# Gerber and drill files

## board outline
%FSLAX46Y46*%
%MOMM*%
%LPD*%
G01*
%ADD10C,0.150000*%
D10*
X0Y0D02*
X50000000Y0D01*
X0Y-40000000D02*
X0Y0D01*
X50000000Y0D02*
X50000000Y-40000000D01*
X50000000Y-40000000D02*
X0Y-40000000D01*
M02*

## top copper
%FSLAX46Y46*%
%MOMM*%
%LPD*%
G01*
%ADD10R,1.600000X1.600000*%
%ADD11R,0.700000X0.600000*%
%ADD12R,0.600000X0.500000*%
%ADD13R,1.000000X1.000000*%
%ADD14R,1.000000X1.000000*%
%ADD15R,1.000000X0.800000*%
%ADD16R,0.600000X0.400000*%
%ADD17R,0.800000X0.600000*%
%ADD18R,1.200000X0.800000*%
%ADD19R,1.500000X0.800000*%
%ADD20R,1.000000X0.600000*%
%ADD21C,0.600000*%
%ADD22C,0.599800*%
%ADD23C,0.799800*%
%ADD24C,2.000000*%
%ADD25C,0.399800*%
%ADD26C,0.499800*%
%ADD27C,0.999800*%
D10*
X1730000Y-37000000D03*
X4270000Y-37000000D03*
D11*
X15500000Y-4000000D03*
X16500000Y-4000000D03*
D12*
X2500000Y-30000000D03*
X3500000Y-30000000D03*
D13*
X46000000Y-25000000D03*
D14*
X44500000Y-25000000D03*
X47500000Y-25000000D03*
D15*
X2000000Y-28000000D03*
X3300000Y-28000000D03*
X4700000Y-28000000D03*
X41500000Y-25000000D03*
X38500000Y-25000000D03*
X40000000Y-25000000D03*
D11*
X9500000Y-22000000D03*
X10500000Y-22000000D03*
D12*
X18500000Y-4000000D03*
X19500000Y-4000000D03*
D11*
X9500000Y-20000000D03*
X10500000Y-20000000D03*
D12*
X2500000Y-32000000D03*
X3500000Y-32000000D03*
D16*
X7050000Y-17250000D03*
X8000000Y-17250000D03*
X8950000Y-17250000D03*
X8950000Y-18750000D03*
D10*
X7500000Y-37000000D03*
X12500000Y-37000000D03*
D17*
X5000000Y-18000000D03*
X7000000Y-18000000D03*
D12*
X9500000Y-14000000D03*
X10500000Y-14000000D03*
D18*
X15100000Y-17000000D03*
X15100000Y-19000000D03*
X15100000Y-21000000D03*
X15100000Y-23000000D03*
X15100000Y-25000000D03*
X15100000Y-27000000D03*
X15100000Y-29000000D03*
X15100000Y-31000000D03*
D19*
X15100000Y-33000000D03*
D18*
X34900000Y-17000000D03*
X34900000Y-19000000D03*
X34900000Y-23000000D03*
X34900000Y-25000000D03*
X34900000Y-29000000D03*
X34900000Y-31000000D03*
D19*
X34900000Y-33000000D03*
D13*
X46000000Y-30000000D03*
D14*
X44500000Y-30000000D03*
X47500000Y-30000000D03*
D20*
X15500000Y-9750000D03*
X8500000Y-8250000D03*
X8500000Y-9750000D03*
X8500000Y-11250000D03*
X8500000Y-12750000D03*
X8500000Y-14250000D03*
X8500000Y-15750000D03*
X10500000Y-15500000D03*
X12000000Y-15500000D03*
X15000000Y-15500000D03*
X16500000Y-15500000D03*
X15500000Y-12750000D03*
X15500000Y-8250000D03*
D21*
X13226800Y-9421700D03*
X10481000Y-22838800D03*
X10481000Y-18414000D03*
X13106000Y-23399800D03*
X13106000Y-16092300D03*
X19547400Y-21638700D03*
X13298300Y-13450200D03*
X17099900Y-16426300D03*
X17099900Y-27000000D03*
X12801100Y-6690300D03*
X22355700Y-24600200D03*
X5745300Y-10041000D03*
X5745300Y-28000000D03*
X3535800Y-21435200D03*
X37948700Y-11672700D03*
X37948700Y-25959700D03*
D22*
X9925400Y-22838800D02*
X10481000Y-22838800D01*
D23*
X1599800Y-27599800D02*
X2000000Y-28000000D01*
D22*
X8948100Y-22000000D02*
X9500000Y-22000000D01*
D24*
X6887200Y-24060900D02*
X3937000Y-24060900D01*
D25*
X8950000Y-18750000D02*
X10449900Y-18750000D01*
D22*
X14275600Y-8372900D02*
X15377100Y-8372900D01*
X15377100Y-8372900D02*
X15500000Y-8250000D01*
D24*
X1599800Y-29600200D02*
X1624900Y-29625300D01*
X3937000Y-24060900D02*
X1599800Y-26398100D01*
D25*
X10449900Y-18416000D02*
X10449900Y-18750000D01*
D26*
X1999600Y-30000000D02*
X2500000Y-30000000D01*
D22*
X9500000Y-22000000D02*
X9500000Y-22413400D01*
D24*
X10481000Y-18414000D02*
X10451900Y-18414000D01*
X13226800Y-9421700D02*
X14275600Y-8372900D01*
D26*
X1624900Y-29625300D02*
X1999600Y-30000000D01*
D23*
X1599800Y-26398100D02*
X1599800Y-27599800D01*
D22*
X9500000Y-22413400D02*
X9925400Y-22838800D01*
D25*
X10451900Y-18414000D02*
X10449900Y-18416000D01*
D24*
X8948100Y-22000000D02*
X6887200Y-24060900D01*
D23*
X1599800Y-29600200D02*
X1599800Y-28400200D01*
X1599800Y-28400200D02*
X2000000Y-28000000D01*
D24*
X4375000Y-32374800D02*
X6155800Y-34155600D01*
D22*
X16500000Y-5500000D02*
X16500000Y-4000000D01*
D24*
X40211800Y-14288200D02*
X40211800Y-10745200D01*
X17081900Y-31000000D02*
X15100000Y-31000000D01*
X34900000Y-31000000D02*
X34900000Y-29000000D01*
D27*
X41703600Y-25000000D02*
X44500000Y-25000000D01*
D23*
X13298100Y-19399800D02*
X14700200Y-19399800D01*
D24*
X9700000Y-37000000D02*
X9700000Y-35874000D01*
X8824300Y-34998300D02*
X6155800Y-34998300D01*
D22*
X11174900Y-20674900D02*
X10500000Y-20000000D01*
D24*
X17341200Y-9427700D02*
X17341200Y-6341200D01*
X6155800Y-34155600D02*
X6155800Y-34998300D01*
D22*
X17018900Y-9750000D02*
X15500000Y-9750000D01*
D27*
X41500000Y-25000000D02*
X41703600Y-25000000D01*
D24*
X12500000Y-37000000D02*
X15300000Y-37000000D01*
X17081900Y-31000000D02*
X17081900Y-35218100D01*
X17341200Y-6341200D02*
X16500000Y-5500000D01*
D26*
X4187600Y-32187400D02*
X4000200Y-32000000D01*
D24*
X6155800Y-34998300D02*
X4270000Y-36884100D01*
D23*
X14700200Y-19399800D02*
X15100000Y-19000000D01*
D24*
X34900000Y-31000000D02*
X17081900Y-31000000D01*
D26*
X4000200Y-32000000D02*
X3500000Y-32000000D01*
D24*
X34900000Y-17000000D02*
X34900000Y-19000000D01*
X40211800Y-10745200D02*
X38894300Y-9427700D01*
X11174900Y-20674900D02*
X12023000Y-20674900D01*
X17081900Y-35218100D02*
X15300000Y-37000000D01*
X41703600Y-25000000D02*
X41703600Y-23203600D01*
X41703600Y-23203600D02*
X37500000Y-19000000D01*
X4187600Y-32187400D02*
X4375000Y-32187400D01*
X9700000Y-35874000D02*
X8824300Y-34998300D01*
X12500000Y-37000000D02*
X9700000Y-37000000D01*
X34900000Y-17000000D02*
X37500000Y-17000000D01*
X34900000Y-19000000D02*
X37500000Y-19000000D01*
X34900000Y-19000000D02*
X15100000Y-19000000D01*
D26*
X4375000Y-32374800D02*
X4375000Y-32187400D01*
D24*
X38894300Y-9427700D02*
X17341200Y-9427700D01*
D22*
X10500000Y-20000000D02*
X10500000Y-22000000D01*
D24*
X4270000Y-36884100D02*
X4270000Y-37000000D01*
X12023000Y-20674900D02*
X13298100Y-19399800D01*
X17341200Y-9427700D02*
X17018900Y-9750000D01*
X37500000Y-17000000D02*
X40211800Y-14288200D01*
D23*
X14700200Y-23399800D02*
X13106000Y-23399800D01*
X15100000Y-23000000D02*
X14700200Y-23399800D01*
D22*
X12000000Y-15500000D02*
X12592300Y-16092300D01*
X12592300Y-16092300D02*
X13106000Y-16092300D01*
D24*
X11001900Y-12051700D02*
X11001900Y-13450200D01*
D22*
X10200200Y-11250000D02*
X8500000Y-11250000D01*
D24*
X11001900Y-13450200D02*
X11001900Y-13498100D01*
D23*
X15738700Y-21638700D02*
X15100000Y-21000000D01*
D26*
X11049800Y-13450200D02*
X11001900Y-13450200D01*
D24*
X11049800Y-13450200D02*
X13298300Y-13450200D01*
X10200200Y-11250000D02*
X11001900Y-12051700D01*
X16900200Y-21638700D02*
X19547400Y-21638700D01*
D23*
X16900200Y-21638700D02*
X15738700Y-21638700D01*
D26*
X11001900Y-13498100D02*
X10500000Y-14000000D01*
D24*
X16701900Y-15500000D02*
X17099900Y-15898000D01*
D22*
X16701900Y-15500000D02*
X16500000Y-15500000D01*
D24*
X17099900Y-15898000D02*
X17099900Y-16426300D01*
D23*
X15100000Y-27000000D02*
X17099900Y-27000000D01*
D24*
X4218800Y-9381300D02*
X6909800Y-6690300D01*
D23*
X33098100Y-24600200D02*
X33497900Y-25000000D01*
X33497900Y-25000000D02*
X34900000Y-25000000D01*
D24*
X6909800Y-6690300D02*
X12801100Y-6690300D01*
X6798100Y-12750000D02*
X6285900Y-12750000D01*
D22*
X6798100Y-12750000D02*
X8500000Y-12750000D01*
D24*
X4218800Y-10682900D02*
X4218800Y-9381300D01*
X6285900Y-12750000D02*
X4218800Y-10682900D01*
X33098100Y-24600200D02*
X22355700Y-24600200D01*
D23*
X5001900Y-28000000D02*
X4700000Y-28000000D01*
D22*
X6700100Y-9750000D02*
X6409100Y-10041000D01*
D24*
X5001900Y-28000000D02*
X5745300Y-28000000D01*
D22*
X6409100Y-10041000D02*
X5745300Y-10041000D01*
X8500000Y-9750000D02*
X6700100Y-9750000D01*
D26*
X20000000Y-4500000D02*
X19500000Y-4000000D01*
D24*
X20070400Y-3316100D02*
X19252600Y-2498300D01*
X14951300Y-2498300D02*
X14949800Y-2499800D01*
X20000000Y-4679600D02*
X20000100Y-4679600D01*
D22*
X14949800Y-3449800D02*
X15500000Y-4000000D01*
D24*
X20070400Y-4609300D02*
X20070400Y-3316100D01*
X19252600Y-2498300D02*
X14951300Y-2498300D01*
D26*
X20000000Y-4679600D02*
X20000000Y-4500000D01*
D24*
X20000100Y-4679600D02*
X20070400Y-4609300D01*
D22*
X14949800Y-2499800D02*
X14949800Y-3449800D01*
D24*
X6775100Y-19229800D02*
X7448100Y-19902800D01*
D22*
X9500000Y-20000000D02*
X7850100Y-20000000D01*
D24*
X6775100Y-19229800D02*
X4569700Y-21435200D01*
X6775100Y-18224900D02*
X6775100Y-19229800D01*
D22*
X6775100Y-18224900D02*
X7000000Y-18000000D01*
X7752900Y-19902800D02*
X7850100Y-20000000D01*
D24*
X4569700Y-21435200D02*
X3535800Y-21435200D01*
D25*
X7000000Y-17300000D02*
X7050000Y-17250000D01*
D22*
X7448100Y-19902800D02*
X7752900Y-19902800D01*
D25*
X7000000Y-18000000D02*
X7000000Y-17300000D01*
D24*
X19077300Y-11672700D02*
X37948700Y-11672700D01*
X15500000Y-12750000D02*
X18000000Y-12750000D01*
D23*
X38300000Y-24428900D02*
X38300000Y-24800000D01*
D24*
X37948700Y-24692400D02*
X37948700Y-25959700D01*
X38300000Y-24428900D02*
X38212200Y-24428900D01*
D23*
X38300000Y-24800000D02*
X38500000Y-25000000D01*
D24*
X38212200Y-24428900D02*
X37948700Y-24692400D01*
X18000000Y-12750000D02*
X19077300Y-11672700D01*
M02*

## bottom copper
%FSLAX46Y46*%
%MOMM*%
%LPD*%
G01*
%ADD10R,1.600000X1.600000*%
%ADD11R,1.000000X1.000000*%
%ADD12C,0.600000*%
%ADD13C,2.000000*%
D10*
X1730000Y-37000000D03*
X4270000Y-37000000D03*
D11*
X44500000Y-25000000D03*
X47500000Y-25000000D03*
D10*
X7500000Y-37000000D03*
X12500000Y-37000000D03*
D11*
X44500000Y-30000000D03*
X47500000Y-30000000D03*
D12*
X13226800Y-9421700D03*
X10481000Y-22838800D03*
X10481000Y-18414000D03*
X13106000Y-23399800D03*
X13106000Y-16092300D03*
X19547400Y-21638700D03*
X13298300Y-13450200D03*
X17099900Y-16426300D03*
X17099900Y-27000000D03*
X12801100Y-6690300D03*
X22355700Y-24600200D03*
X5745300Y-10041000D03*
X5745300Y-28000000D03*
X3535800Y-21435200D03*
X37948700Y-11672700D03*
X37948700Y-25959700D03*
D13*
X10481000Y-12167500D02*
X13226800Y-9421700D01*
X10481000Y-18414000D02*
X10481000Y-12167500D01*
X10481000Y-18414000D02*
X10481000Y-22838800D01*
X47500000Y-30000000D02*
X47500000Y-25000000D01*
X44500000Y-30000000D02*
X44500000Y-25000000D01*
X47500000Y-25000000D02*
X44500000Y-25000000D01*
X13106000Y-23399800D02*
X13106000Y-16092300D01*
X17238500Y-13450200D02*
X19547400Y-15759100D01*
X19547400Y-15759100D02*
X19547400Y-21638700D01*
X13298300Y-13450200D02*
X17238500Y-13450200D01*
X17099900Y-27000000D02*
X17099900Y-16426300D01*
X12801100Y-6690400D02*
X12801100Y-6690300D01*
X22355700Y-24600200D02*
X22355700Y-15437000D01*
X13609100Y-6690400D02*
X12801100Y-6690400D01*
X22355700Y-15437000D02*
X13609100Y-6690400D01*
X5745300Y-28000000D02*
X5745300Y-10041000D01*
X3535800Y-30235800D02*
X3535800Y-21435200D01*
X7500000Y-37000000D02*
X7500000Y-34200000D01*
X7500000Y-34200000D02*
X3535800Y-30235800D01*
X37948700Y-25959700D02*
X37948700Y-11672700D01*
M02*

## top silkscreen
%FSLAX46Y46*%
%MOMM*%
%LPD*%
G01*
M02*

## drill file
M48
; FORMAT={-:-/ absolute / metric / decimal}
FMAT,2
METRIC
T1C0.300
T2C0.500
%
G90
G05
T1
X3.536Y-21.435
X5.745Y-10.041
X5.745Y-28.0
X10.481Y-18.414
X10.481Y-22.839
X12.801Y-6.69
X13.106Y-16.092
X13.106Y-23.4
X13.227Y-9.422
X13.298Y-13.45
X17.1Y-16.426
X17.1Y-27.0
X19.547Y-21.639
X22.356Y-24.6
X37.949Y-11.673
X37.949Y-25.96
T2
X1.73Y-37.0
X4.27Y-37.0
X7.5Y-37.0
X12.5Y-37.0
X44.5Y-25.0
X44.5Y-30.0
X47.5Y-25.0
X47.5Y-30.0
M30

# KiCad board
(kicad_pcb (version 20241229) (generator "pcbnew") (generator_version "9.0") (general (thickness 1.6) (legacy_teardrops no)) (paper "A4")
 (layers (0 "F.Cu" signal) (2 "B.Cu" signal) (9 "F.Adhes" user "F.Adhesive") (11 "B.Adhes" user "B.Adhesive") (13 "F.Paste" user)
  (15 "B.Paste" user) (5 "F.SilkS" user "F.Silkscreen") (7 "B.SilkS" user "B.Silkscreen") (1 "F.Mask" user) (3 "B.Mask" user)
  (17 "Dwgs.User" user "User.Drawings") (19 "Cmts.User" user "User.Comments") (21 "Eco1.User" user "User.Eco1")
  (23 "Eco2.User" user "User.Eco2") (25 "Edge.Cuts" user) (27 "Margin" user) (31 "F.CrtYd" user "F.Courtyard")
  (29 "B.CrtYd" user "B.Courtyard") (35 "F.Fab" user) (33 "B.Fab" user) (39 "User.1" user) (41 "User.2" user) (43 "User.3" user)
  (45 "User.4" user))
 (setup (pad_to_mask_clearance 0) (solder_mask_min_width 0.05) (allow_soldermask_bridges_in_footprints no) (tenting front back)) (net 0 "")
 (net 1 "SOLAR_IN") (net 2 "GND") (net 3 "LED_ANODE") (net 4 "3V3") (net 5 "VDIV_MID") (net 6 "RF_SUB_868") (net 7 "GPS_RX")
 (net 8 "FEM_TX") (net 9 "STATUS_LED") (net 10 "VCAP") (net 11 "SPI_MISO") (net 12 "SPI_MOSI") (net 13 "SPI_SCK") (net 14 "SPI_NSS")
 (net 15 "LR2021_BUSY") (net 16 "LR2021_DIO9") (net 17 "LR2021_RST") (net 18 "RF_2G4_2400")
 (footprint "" (layer "F.Cu") (at 3 37)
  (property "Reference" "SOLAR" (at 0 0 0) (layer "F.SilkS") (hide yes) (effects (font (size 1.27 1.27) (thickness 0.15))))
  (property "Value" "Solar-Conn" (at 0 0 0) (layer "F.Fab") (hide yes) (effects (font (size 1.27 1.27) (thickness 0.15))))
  (pad "1" thru_hole rect (at -1.27 0) (size 1.6 1.6) (drill 0.5) (layers "*.Cu" "*.Mask") (remove_unused_layers no) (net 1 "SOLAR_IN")
   (thermal_bridge_angle 45))
  (pad "2" thru_hole rect (at 1.27 0) (size 1.6 1.6) (drill 0.5) (layers "*.Cu" "*.Mask") (remove_unused_layers no) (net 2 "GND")
   (thermal_bridge_angle 45)))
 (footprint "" (layer "F.Cu") (at 16 4)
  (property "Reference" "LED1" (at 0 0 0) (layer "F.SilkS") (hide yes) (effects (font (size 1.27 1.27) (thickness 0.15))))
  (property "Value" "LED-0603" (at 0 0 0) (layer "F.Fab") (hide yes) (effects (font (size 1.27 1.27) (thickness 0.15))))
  (pad "A" smd rect (at -0.5 0) (size 0.7 0.6) (layers "F.Cu" "F.Mask") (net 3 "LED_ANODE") (thermal_bridge_angle 45))
  (pad "K" smd rect (at 0.5 0) (size 0.7 0.6) (layers "F.Cu" "F.Mask") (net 2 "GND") (thermal_bridge_angle 45)))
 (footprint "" (layer "F.Cu") (at 3 30)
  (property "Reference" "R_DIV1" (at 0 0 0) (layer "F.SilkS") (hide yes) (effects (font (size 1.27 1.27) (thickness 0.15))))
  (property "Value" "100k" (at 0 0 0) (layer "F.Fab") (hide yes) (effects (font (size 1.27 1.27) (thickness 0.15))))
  (pad "1" smd rect (at -0.5 0) (size 0.6 0.5) (layers "F.Cu" "F.Mask") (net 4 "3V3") (thermal_bridge_angle 45))
  (pad "2" smd rect (at 0.5 0) (size 0.6 0.5) (layers "F.Cu" "F.Mask") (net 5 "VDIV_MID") (thermal_bridge_angle 45)))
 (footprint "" (layer "F.Cu") (at 46 25)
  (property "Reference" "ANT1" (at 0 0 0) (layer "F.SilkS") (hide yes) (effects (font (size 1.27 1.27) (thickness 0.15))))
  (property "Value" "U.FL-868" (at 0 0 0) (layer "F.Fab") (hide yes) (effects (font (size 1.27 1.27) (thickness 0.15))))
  (pad "1" smd rect (at 0 0) (size 1 1) (layers "F.Cu" "F.Mask") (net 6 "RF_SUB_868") (thermal_bridge_angle 45))
  (pad "2" thru_hole rect (at -1.5 0) (size 1 1) (drill 0.5) (layers "*.Cu" "*.Mask") (remove_unused_layers no) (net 2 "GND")
   (thermal_bridge_angle 45))
  (pad "3" thru_hole rect (at 1.5 0) (size 1 1) (drill 0.5) (layers "*.Cu" "*.Mask") (remove_unused_layers no) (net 2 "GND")
   (thermal_bridge_angle 45)))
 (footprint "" (layer "F.Cu") (at 4 28)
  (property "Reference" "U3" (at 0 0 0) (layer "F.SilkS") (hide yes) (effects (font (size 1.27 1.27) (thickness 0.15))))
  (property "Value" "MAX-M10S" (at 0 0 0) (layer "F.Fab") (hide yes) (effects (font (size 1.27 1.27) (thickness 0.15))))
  (pad "1" smd rect (at -2 0) (size 1 0.8) (layers "F.Cu" "F.Mask") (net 4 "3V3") (thermal_bridge_angle 45))
  (pad "2" smd rect (at -0.7 0) (size 1 0.8) (layers "F.Cu" "F.Mask") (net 2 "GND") (thermal_bridge_angle 45))
  (pad "3" smd rect (at 0.7 0) (size 1 0.8) (layers "F.Cu" "F.Mask") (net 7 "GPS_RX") (thermal_bridge_angle 45)))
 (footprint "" (layer "F.Cu") (at 40 25)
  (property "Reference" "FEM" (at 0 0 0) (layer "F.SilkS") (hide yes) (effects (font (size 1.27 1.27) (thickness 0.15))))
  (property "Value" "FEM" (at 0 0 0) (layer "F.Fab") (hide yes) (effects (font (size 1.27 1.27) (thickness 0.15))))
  (pad "GND" smd rect (at 1.5 0) (size 1 0.8) (layers "F.Cu" "F.Mask") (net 2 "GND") (thermal_bridge_angle 45))
  (pad "TX" smd rect (at -1.5 0) (size 1 0.8) (layers "F.Cu" "F.Mask") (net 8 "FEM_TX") (thermal_bridge_angle 45))
  (pad "VCC" smd rect (at 0 0) (size 1 0.8) (layers "F.Cu" "F.Mask") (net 4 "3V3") (thermal_bridge_angle 45)))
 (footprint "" (layer "F.Cu") (at 10 22)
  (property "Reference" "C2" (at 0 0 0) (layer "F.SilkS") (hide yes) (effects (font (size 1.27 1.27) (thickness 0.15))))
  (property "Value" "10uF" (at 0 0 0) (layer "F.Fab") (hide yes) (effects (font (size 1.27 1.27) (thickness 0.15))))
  (pad "1" smd rect (at -0.5 0) (size 0.7 0.6) (layers "F.Cu" "F.Mask") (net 4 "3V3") (thermal_bridge_angle 45))
  (pad "2" smd rect (at 0.5 0) (size 0.7 0.6) (layers "F.Cu" "F.Mask") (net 2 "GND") (thermal_bridge_angle 45)))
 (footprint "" (layer "F.Cu") (at 19 4)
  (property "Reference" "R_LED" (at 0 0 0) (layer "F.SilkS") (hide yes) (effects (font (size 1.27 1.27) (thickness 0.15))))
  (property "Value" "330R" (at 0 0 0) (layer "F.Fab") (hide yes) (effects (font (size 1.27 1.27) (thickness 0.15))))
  (pad "1" smd rect (at -0.5 0) (size 0.6 0.5) (layers "F.Cu" "F.Mask") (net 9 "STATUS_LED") (thermal_bridge_angle 45))
  (pad "2" smd rect (at 0.5 0) (size 0.6 0.5) (layers "F.Cu" "F.Mask") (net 3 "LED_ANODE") (thermal_bridge_angle 45)))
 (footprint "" (layer "F.Cu") (at 10 20)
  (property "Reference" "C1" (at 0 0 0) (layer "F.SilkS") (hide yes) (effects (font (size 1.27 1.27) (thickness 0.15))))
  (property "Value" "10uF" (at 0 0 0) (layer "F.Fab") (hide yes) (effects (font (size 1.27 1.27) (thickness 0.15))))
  (pad "1" smd rect (at -0.5 0) (size 0.7 0.6) (layers "F.Cu" "F.Mask") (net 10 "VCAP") (thermal_bridge_angle 45))
  (pad "2" smd rect (at 0.5 0) (size 0.7 0.6) (layers "F.Cu" "F.Mask") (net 2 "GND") (thermal_bridge_angle 45)))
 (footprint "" (layer "F.Cu") (at 3 32)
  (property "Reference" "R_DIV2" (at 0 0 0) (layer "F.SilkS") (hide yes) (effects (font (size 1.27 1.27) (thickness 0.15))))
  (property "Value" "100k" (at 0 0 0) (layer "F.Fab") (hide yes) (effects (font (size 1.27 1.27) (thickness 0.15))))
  (pad "1" smd rect (at -0.5 0) (size 0.6 0.5) (layers "F.Cu" "F.Mask") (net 5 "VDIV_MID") (thermal_bridge_angle 45))
  (pad "2" smd rect (at 0.5 0) (size 0.6 0.5) (layers "F.Cu" "F.Mask") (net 2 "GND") (thermal_bridge_angle 45)))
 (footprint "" (layer "F.Cu") (at 8 18)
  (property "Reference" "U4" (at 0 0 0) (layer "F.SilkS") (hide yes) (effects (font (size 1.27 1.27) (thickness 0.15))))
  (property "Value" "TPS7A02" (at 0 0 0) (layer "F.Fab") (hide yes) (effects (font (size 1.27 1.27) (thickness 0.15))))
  (pad "1" smd rect (at -0.95 -0.75) (size 0.6 0.4) (layers "F.Cu" "F.Mask") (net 10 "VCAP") (thermal_bridge_angle 45))
  (pad "2" smd rect (at 0 -0.75) (size 0.6 0.4) (layers "F.Cu" "F.Mask") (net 2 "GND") (thermal_bridge_angle 45))
  (pad "3" smd rect (at 0.95 -0.75) (size 0.6 0.4) (layers "F.Cu" "F.Mask") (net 10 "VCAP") (thermal_bridge_angle 45))
  (pad "4" smd rect (at 0.95 0.75) (size 0.6 0.4) (layers "F.Cu" "F.Mask") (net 4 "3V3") (thermal_bridge_angle 45)))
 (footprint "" (layer "F.Cu") (at 10 37)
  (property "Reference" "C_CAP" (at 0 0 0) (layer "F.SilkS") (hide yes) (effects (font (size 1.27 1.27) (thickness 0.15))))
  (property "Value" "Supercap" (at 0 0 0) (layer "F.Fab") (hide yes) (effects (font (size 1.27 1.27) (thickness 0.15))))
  (pad "1" thru_hole rect (at -2.5 0) (size 1.6 1.6) (drill 0.5) (layers "*.Cu" "*.Mask") (remove_unused_layers no) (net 10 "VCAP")
   (thermal_bridge_angle 45))
  (pad "2" thru_hole rect (at 2.5 0) (size 1.6 1.6) (drill 0.5) (layers "*.Cu" "*.Mask") (remove_unused_layers no) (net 2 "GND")
   (thermal_bridge_angle 45)))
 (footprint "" (layer "F.Cu") (at 6 18)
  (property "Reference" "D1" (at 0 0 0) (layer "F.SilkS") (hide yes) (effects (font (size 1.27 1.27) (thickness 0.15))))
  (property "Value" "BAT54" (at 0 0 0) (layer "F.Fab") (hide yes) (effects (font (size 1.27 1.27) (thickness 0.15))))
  (pad "A" smd rect (at -1 0) (size 0.8 0.6) (layers "F.Cu" "F.Mask") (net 1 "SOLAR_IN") (thermal_bridge_angle 45))
  (pad "K" smd rect (at 1 0) (size 0.8 0.6) (layers "F.Cu" "F.Mask") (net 10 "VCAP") (thermal_bridge_angle 45)))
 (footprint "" (layer "F.Cu") (at 10 14)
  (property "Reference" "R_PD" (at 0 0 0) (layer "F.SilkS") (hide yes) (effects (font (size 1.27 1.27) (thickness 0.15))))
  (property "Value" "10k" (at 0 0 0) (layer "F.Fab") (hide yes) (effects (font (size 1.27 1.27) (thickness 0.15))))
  (pad "1" smd rect (at -0.5 0) (size 0.6 0.5) (layers "F.Cu" "F.Mask") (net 2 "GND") (thermal_bridge_angle 45))
  (pad "2" smd rect (at 0.5 0) (size 0.6 0.5) (layers "F.Cu" "F.Mask") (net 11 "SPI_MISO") (thermal_bridge_angle 45)))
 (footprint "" (layer "F.Cu") (at 25 25)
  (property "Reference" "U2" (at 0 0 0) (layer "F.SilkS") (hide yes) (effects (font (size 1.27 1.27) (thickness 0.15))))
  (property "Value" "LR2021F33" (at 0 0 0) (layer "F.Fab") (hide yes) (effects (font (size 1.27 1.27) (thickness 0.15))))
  (pad "1" smd rect (at -9.9 -8) (size 1.2 0.8) (layers "F.Cu" "F.Mask") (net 4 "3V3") (thermal_bridge_angle 45))
  (pad "2" smd rect (at -9.9 -6) (size 1.2 0.8) (layers "F.Cu" "F.Mask") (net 2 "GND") (thermal_bridge_angle 45))
  (pad "3" smd rect (at -9.9 -4) (size 1.2 0.8) (layers "F.Cu" "F.Mask") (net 11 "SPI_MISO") (thermal_bridge_angle 45))
  (pad "4" smd rect (at -9.9 -2) (size 1.2 0.8) (layers "F.Cu" "F.Mask") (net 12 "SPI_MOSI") (thermal_bridge_angle 45))
  (pad "5" smd rect (at -9.9 0) (size 1.2 0.8) (layers "F.Cu" "F.Mask") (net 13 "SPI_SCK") (thermal_bridge_angle 45))
  (pad "6" smd rect (at -9.9 2) (size 1.2 0.8) (layers "F.Cu" "F.Mask") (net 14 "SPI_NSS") (thermal_bridge_angle 45))
  (pad "7" smd rect (at -9.9 4) (size 1.2 0.8) (layers "F.Cu" "F.Mask") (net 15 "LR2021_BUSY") (thermal_bridge_angle 45))
  (pad "8" smd rect (at -9.9 6) (size 1.2 0.8) (layers "F.Cu" "F.Mask") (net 2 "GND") (thermal_bridge_angle 45))
  (pad "9" smd rect (at -9.9 8) (size 1.5 0.8) (layers "F.Cu" "F.Mask") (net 6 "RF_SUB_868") (thermal_bridge_angle 45))
  (pad "10" smd rect (at 9.9 -8) (size 1.2 0.8) (layers "F.Cu" "F.Mask") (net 2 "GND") (thermal_bridge_angle 45))
  (pad "11" smd rect (at 9.9 -6) (size 1.2 0.8) (layers "F.Cu" "F.Mask") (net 2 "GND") (thermal_bridge_angle 45))
  (pad "13" smd rect (at 9.9 -2) (size 1.2 0.8) (layers "F.Cu" "F.Mask") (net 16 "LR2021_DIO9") (thermal_bridge_angle 45))
  (pad "14" smd rect (at 9.9 0) (size 1.2 0.8) (layers "F.Cu" "F.Mask") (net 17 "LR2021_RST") (thermal_bridge_angle 45))
  (pad "16" smd rect (at 9.9 4) (size 1.2 0.8) (layers "F.Cu" "F.Mask") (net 2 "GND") (thermal_bridge_angle 45))
  (pad "17" smd rect (at 9.9 6) (size 1.2 0.8) (layers "F.Cu" "F.Mask") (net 2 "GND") (thermal_bridge_angle 45))
  (pad "18" smd rect (at 9.9 8) (size 1.5 0.8) (layers "F.Cu" "F.Mask") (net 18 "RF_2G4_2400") (thermal_bridge_angle 45)))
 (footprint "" (layer "F.Cu") (at 46 30)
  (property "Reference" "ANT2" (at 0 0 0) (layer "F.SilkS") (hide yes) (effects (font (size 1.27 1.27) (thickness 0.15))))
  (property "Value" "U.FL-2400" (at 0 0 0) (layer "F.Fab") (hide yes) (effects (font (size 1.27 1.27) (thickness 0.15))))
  (pad "1" smd rect (at 0 0) (size 1 1) (layers "F.Cu" "F.Mask") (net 18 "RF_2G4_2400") (thermal_bridge_angle 45))
  (pad "2" thru_hole rect (at -1.5 0) (size 1 1) (drill 0.5) (layers "*.Cu" "*.Mask") (remove_unused_layers no) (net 2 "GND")
   (thermal_bridge_angle 45))
  (pad "3" thru_hole rect (at 1.5 0) (size 1 1) (drill 0.5) (layers "*.Cu" "*.Mask") (remove_unused_layers no) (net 2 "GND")
   (thermal_bridge_angle 45)))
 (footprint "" (layer "F.Cu") (at 12 12)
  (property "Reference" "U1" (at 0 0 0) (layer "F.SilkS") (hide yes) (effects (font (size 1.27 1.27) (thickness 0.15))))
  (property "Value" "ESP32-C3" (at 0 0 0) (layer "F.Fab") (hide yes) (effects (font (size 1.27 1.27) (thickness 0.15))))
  (pad "GND" smd rect (at 3.5 -2.25) (size 1 0.6) (layers "F.Cu" "F.Mask") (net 2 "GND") (thermal_bridge_angle 45))
  (pad "GPIO0" smd rect (at -3.5 -3.75) (size 1 0.6) (layers "F.Cu" "F.Mask") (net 5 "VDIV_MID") (thermal_bridge_angle 45))
  (pad "GPIO1" smd rect (at -3.5 -2.25) (size 1 0.6) (layers "F.Cu" "F.Mask") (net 7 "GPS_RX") (thermal_bridge_angle 45))
  (pad "GPIO2" smd rect (at -3.5 -0.75) (size 1 0.6) (layers "F.Cu" "F.Mask") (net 11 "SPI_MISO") (thermal_bridge_angle 45))
  (pad "GPIO3" smd rect (at -3.5 0.75) (size 1 0.6) (layers "F.Cu" "F.Mask") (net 17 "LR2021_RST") (thermal_bridge_angle 45))
  (pad "GPIO4" smd rect (at -3.5 2.25) (size 1 0.6) (layers "F.Cu" "F.Mask") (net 15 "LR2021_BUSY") (thermal_bridge_angle 45))
  (pad "GPIO5" smd rect (at -3.5 3.75) (size 1 0.6) (layers "F.Cu" "F.Mask") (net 16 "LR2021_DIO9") (thermal_bridge_angle 45))
  (pad "GPIO6" smd rect (at -1.5 3.5) (size 1 0.6) (layers "F.Cu" "F.Mask") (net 13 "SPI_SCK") (thermal_bridge_angle 45))
  (pad "GPIO7" smd rect (at 0 3.5) (size 1 0.6) (layers "F.Cu" "F.Mask") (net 12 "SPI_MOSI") (thermal_bridge_angle 45))
  (pad "GPIO9" smd rect (at 3 3.5) (size 1 0.6) (layers "F.Cu" "F.Mask") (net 9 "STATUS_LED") (thermal_bridge_angle 45))
  (pad "GPIO10" smd rect (at 4.5 3.5) (size 1 0.6) (layers "F.Cu" "F.Mask") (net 14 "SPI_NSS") (thermal_bridge_angle 45))
  (pad "GPIO19" smd rect (at 3.5 0.75) (size 1 0.6) (layers "F.Cu" "F.Mask") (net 8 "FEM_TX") (thermal_bridge_angle 45))
  (pad "VCC" smd rect (at 3.5 -3.75) (size 1 0.6) (layers "F.Cu" "F.Mask") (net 4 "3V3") (thermal_bridge_angle 45)))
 (gr_line (start 0 0) (end 50 0) (stroke (width 0.15) (type default)) (layer "Edge.Cuts"))
 (gr_line (start 0 40) (end 0 0) (stroke (width 0.15) (type default)) (layer "Edge.Cuts"))
 (gr_line (start 50 0) (end 50 40) (stroke (width 0.15) (type default)) (layer "Edge.Cuts"))
 (gr_line (start 50 40) (end 0 40) (stroke (width 0.15) (type default)) (layer "Edge.Cuts"))
 (segment (start 9.9254 22.8388) (end 10.481 22.8388) (width 0.5998) (layer "F.Cu") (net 4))
 (segment (start 1.5998 27.5998) (end 2 28) (width 0.7998) (layer "F.Cu") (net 4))
 (segment (start 8.9481 22) (end 9.5 22) (width 0.5998) (layer "F.Cu") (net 4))
 (segment (start 6.8872 24.0609) (end 3.937 24.0609) (width 2) (layer "F.Cu") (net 4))
 (segment (start 8.95 18.75) (end 10.4499 18.75) (width 0.3998) (layer "F.Cu") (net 4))
 (segment (start 14.2756 8.3729) (end 15.3771 8.3729) (width 0.5998) (layer "F.Cu") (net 4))
 (segment (start 15.3771 8.3729) (end 15.5 8.25) (width 0.5998) (layer "F.Cu") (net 4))
 (segment (start 1.5998 29.6002) (end 1.6249 29.6253) (width 2) (layer "F.Cu") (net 4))
 (segment (start 3.937 24.0609) (end 1.5998 26.3981) (width 2) (layer "F.Cu") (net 4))
 (segment (start 10.4499 18.416) (end 10.4499 18.75) (width 0.3998) (layer "F.Cu") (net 4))
 (segment (start 1.9996 30) (end 2.5 30) (width 0.4998) (layer "F.Cu") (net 4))
 (segment (start 9.5 22) (end 9.5 22.4134) (width 0.5998) (layer "F.Cu") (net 4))
 (segment (start 10.481 18.414) (end 10.4519 18.414) (width 2) (layer "F.Cu") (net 4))
 (segment (start 13.2268 9.4217) (end 14.2756 8.3729) (width 2) (layer "F.Cu") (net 4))
 (segment (start 1.6249 29.6253) (end 1.9996 30) (width 0.4998) (layer "F.Cu") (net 4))
 (segment (start 1.5998 26.3981) (end 1.5998 27.5998) (width 0.7998) (layer "F.Cu") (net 4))
 (segment (start 9.5 22.4134) (end 9.9254 22.8388) (width 0.5998) (layer "F.Cu") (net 4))
 (segment (start 10.4519 18.414) (end 10.4499 18.416) (width 0.3998) (layer "F.Cu") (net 4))
 (segment (start 8.9481 22) (end 6.8872 24.0609) (width 2) (layer "F.Cu") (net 4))
 (segment (start 1.5998 29.6002) (end 1.5998 28.4002) (width 0.7998) (layer "F.Cu") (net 4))
 (segment (start 1.5998 28.4002) (end 2 28) (width 0.7998) (layer "F.Cu") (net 4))
 (via (at 13.2268 9.4217) (size 0.6) (drill 0.3) (layers "F.Cu" "B.Cu") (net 4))
 (via (at 10.481 22.8388) (size 0.6) (drill 0.3) (layers "F.Cu" "B.Cu") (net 4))
 (via (at 10.481 18.414) (size 0.6) (drill 0.3) (layers "F.Cu" "B.Cu") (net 4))
 (segment (start 10.481 12.1675) (end 13.2268 9.4217) (width 2) (layer "B.Cu") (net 4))
 (segment (start 10.481 18.414) (end 10.481 12.1675) (width 2) (layer "B.Cu") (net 4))
 (segment (start 10.481 18.414) (end 10.481 22.8388) (width 2) (layer "B.Cu") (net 4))
 (segment (start 4.375 32.3748) (end 6.1558 34.1556) (width 2) (layer "F.Cu") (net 2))
 (segment (start 16.5 5.5) (end 16.5 4) (width 0.5998) (layer "F.Cu") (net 2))
 (segment (start 40.2118 14.2882) (end 40.2118 10.7452) (width 2) (layer "F.Cu") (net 2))
 (segment (start 17.0819 31) (end 15.1 31) (width 2) (layer "F.Cu") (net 2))
 (segment (start 34.9 31) (end 34.9 29) (width 2) (layer "F.Cu") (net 2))
 (segment (start 41.7036 25) (end 44.5 25) (width 0.9998) (layer "F.Cu") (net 2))
 (segment (start 13.2981 19.3998) (end 14.7002 19.3998) (width 0.7998) (layer "F.Cu") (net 2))
 (segment (start 9.7 37) (end 9.7 35.874) (width 2) (layer "F.Cu") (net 2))
 (segment (start 8.8243 34.9983) (end 6.1558 34.9983) (width 2) (layer "F.Cu") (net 2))
 (segment (start 11.1749 20.6749) (end 10.5 20) (width 0.5998) (layer "F.Cu") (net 2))
 (segment (start 17.3412 9.4277) (end 17.3412 6.3412) (width 2) (layer "F.Cu") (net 2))
 (segment (start 6.1558 34.1556) (end 6.1558 34.9983) (width 2) (layer "F.Cu") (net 2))
 (segment (start 17.0189 9.75) (end 15.5 9.75) (width 0.5998) (layer "F.Cu") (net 2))
 (segment (start 41.5 25) (end 41.7036 25) (width 0.9998) (layer "F.Cu") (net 2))
 (segment (start 12.5 37) (end 15.3 37) (width 2) (layer "F.Cu") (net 2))
 (segment (start 17.0819 31) (end 17.0819 35.2181) (width 2) (layer "F.Cu") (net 2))
 (segment (start 17.3412 6.3412) (end 16.5 5.5) (width 2) (layer "F.Cu") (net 2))
 (segment (start 4.1876 32.1874) (end 4.0002 32) (width 0.4998) (layer "F.Cu") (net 2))
 (segment (start 6.1558 34.9983) (end 4.27 36.8841) (width 2) (layer "F.Cu") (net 2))
 (segment (start 14.7002 19.3998) (end 15.1 19) (width 0.7998) (layer "F.Cu") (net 2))
 (segment (start 34.9 31) (end 17.0819 31) (width 2) (layer "F.Cu") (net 2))
 (segment (start 4.0002 32) (end 3.5 32) (width 0.4998) (layer "F.Cu") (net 2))
 (segment (start 34.9 17) (end 34.9 19) (width 2) (layer "F.Cu") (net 2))
 (segment (start 40.2118 10.7452) (end 38.8943 9.4277) (width 2) (layer "F.Cu") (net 2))
 (segment (start 11.1749 20.6749) (end 12.023 20.6749) (width 2) (layer "F.Cu") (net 2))
 (segment (start 17.0819 35.2181) (end 15.3 37) (width 2) (layer "F.Cu") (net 2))
 (segment (start 41.7036 25) (end 41.7036 23.2036) (width 2) (layer "F.Cu") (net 2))
 (segment (start 41.7036 23.2036) (end 37.5 19) (width 2) (layer "F.Cu") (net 2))
 (segment (start 4.1876 32.1874) (end 4.375 32.1874) (width 2) (layer "F.Cu") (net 2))
 (segment (start 9.7 35.874) (end 8.8243 34.9983) (width 2) (layer "F.Cu") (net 2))
 (segment (start 12.5 37) (end 9.7 37) (width 2) (layer "F.Cu") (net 2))
 (segment (start 34.9 17) (end 37.5 17) (width 2) (layer "F.Cu") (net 2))
 (segment (start 34.9 19) (end 37.5 19) (width 2) (layer "F.Cu") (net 2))
 (segment (start 34.9 19) (end 15.1 19) (width 2) (layer "F.Cu") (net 2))
 (segment (start 4.375 32.3748) (end 4.375 32.1874) (width 0.4998) (layer "F.Cu") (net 2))
 (segment (start 38.8943 9.4277) (end 17.3412 9.4277) (width 2) (layer "F.Cu") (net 2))
 (segment (start 10.5 20) (end 10.5 22) (width 0.5998) (layer "F.Cu") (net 2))
 (segment (start 4.27 36.8841) (end 4.27 37) (width 2) (layer "F.Cu") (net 2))
 (segment (start 12.023 20.6749) (end 13.2981 19.3998) (width 2) (layer "F.Cu") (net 2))
 (segment (start 17.3412 9.4277) (end 17.0189 9.75) (width 2) (layer "F.Cu") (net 2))
 (segment (start 37.5 17) (end 40.2118 14.2882) (width 2) (layer "F.Cu") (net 2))
 (segment (start 47.5 30) (end 47.5 25) (width 2) (layer "B.Cu") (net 2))
 (segment (start 44.5 30) (end 44.5 25) (width 2) (layer "B.Cu") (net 2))
 (segment (start 47.5 25) (end 44.5 25) (width 2) (layer "B.Cu") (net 2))
 (segment (start 14.7002 23.3998) (end 13.106 23.3998) (width 0.7998) (layer "F.Cu") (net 12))
 (segment (start 15.1 23) (end 14.7002 23.3998) (width 0.7998) (layer "F.Cu") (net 12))
 (segment (start 12 15.5) (end 12.5923 16.0923) (width 0.5998) (layer "F.Cu") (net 12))
 (segment (start 12.5923 16.0923) (end 13.106 16.0923) (width 0.5998) (layer "F.Cu") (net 12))
 (via (at 13.106 23.3998) (size 0.6) (drill 0.3) (layers "F.Cu" "B.Cu") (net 12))
 (via (at 13.106 16.0923) (size 0.6) (drill 0.3) (layers "F.Cu" "B.Cu") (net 12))
 (segment (start 13.106 23.3998) (end 13.106 16.0923) (width 2) (layer "B.Cu") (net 12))
 (segment (start 11.0019 12.0517) (end 11.0019 13.4502) (width 2) (layer "F.Cu") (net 11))
 (segment (start 10.2002 11.25) (end 8.5 11.25) (width 0.5998) (layer "F.Cu") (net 11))
 (segment (start 11.0019 13.4502) (end 11.0019 13.4981) (width 2) (layer "F.Cu") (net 11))
 (segment (start 15.7387 21.6387) (end 15.1 21) (width 0.7998) (layer "F.Cu") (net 11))
 (segment (start 11.0498 13.4502) (end 11.0019 13.4502) (width 0.4998) (layer "F.Cu") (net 11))
 (segment (start 11.0498 13.4502) (end 13.2983 13.4502) (width 2) (layer "F.Cu") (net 11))
 (segment (start 10.2002 11.25) (end 11.0019 12.0517) (width 2) (layer "F.Cu") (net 11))
 (segment (start 16.9002 21.6387) (end 19.5474 21.6387) (width 2) (layer "F.Cu") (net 11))
 (segment (start 16.9002 21.6387) (end 15.7387 21.6387) (width 0.7998) (layer "F.Cu") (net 11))
 (segment (start 11.0019 13.4981) (end 10.5 14) (width 0.4998) (layer "F.Cu") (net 11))
 (via (at 19.5474 21.6387) (size 0.6) (drill 0.3) (layers "F.Cu" "B.Cu") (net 11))
 (via (at 13.2983 13.4502) (size 0.6) (drill 0.3) (layers "F.Cu" "B.Cu") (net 11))
 (segment (start 17.2385 13.4502) (end 19.5474 15.7591) (width 2) (layer "B.Cu") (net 11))
 (segment (start 19.5474 15.7591) (end 19.5474 21.6387) (width 2) (layer "B.Cu") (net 11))
 (segment (start 13.2983 13.4502) (end 17.2385 13.4502) (width 2) (layer "B.Cu") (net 11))
 (segment (start 16.7019 15.5) (end 17.0999 15.898) (width 2) (layer "F.Cu") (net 14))
 (segment (start 16.7019 15.5) (end 16.5 15.5) (width 0.5998) (layer "F.Cu") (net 14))
 (segment (start 17.0999 15.898) (end 17.0999 16.4263) (width 2) (layer "F.Cu") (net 14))
 (segment (start 15.1 27) (end 17.0999 27) (width 0.7998) (layer "F.Cu") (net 14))
 (via (at 17.0999 16.4263) (size 0.6) (drill 0.3) (layers "F.Cu" "B.Cu") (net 14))
 (via (at 17.0999 27) (size 0.6) (drill 0.3) (layers "F.Cu" "B.Cu") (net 14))
 (segment (start 17.0999 27) (end 17.0999 16.4263) (width 2) (layer "B.Cu") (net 14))
 (segment (start 4.2188 9.3813) (end 6.9098 6.6903) (width 2) (layer "F.Cu") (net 17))
 (segment (start 33.0981 24.6002) (end 33.4979 25) (width 0.7998) (layer "F.Cu") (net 17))
 (segment (start 33.4979 25) (end 34.9 25) (width 0.7998) (layer "F.Cu") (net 17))
 (segment (start 6.9098 6.6903) (end 12.8011 6.6903) (width 2) (layer "F.Cu") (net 17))
 (segment (start 6.7981 12.75) (end 6.2859 12.75) (width 2) (layer "F.Cu") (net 17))
 (segment (start 6.7981 12.75) (end 8.5 12.75) (width 0.5998) (layer "F.Cu") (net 17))
 (segment (start 4.2188 10.6829) (end 4.2188 9.3813) (width 2) (layer "F.Cu") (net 17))
 (segment (start 6.2859 12.75) (end 4.2188 10.6829) (width 2) (layer "F.Cu") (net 17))
 (segment (start 33.0981 24.6002) (end 22.3557 24.6002) (width 2) (layer "F.Cu") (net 17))
 (via (at 12.8011 6.6903) (size 0.6) (drill 0.3) (layers "F.Cu" "B.Cu") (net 17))
 (via (at 22.3557 24.6002) (size 0.6) (drill 0.3) (layers "F.Cu" "B.Cu") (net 17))
 (segment (start 12.8011 6.6904) (end 12.8011 6.6903) (width 2) (layer "B.Cu") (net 17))
 (segment (start 22.3557 24.6002) (end 22.3557 15.437) (width 2) (layer "B.Cu") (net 17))
 (segment (start 13.6091 6.6904) (end 12.8011 6.6904) (width 2) (layer "B.Cu") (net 17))
 (segment (start 22.3557 15.437) (end 13.6091 6.6904) (width 2) (layer "B.Cu") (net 17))
 (segment (start 5.0019 28) (end 4.7 28) (width 0.7998) (layer "F.Cu") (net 7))
 (segment (start 6.7001 9.75) (end 6.4091 10.041) (width 0.5998) (layer "F.Cu") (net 7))
 (segment (start 5.0019 28) (end 5.7453 28) (width 2) (layer "F.Cu") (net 7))
 (segment (start 6.4091 10.041) (end 5.7453 10.041) (width 0.5998) (layer "F.Cu") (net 7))
 (segment (start 8.5 9.75) (end 6.7001 9.75) (width 0.5998) (layer "F.Cu") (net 7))
 (via (at 5.7453 10.041) (size 0.6) (drill 0.3) (layers "F.Cu" "B.Cu") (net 7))
 (via (at 5.7453 28) (size 0.6) (drill 0.3) (layers "F.Cu" "B.Cu") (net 7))
 (segment (start 5.7453 28) (end 5.7453 10.041) (width 2) (layer "B.Cu") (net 7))
 (segment (start 20 4.5) (end 19.5 4) (width 0.4998) (layer "F.Cu") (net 3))
 (segment (start 20.0704 3.3161) (end 19.2526 2.4983) (width 2) (layer "F.Cu") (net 3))
 (segment (start 14.9513 2.4983) (end 14.9498 2.4998) (width 2) (layer "F.Cu") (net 3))
 (segment (start 20 4.6796) (end 20.0001 4.6796) (width 2) (layer "F.Cu") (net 3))
 (segment (start 14.9498 3.4498) (end 15.5 4) (width 0.5998) (layer "F.Cu") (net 3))
 (segment (start 20.0704 4.6093) (end 20.0704 3.3161) (width 2) (layer "F.Cu") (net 3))
 (segment (start 19.2526 2.4983) (end 14.9513 2.4983) (width 2) (layer "F.Cu") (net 3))
 (segment (start 20 4.6796) (end 20 4.5) (width 0.4998) (layer "F.Cu") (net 3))
 (segment (start 20.0001 4.6796) (end 20.0704 4.6093) (width 2) (layer "F.Cu") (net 3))
 (segment (start 14.9498 2.4998) (end 14.9498 3.4498) (width 0.5998) (layer "F.Cu") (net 3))
 (segment (start 6.7751 19.2298) (end 7.4481 19.9028) (width 2) (layer "F.Cu") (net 10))
 (segment (start 9.5 20) (end 7.8501 20) (width 0.5998) (layer "F.Cu") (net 10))
 (segment (start 6.7751 19.2298) (end 4.5697 21.4352) (width 2) (layer "F.Cu") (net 10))
 (segment (start 6.7751 18.2249) (end 6.7751 19.2298) (width 2) (layer "F.Cu") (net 10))
 (segment (start 6.7751 18.2249) (end 7 18) (width 0.5998) (layer "F.Cu") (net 10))
 (segment (start 7.7529 19.9028) (end 7.8501 20) (width 0.5998) (layer "F.Cu") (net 10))
 (segment (start 4.5697 21.4352) (end 3.5358 21.4352) (width 2) (layer "F.Cu") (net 10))
 (segment (start 7 17.3) (end 7.05 17.25) (width 0.3998) (layer "F.Cu") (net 10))
 (segment (start 7.4481 19.9028) (end 7.7529 19.9028) (width 0.5998) (layer "F.Cu") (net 10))
 (segment (start 7 18) (end 7 17.3) (width 0.3998) (layer "F.Cu") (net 10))
 (via (at 3.5358 21.4352) (size 0.6) (drill 0.3) (layers "F.Cu" "B.Cu") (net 10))
 (segment (start 3.5358 30.2358) (end 3.5358 21.4352) (width 2) (layer "B.Cu") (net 10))
 (segment (start 7.5 37) (end 7.5 34.2) (width 2) (layer "B.Cu") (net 10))
 (segment (start 7.5 34.2) (end 3.5358 30.2358) (width 2) (layer "B.Cu") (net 10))
 (segment (start 19.0773 11.6727) (end 37.9487 11.6727) (width 2) (layer "F.Cu") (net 8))
 (segment (start 15.5 12.75) (end 18 12.75) (width 2) (layer "F.Cu") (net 8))
 (segment (start 38.3 24.4289) (end 38.3 24.8) (width 0.7998) (layer "F.Cu") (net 8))
 (segment (start 37.9487 24.6924) (end 37.9487 25.9597) (width 2) (layer "F.Cu") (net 8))
 (segment (start 38.3 24.4289) (end 38.2122 24.4289) (width 2) (layer "F.Cu") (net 8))
 (segment (start 38.3 24.8) (end 38.5 25) (width 0.7998) (layer "F.Cu") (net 8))
 (segment (start 38.2122 24.4289) (end 37.9487 24.6924) (width 2) (layer "F.Cu") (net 8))
 (segment (start 18 12.75) (end 19.0773 11.6727) (width 2) (layer "F.Cu") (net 8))
 (via (at 37.9487 11.6727) (size 0.6) (drill 0.3) (layers "F.Cu" "B.Cu") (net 8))
 (via (at 37.9487 25.9597) (size 0.6) (drill 0.3) (layers "F.Cu" "B.Cu") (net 8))
 (segment (start 37.9487 25.9597) (end 37.9487 11.6727) (width 2) (layer "B.Cu") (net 8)))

